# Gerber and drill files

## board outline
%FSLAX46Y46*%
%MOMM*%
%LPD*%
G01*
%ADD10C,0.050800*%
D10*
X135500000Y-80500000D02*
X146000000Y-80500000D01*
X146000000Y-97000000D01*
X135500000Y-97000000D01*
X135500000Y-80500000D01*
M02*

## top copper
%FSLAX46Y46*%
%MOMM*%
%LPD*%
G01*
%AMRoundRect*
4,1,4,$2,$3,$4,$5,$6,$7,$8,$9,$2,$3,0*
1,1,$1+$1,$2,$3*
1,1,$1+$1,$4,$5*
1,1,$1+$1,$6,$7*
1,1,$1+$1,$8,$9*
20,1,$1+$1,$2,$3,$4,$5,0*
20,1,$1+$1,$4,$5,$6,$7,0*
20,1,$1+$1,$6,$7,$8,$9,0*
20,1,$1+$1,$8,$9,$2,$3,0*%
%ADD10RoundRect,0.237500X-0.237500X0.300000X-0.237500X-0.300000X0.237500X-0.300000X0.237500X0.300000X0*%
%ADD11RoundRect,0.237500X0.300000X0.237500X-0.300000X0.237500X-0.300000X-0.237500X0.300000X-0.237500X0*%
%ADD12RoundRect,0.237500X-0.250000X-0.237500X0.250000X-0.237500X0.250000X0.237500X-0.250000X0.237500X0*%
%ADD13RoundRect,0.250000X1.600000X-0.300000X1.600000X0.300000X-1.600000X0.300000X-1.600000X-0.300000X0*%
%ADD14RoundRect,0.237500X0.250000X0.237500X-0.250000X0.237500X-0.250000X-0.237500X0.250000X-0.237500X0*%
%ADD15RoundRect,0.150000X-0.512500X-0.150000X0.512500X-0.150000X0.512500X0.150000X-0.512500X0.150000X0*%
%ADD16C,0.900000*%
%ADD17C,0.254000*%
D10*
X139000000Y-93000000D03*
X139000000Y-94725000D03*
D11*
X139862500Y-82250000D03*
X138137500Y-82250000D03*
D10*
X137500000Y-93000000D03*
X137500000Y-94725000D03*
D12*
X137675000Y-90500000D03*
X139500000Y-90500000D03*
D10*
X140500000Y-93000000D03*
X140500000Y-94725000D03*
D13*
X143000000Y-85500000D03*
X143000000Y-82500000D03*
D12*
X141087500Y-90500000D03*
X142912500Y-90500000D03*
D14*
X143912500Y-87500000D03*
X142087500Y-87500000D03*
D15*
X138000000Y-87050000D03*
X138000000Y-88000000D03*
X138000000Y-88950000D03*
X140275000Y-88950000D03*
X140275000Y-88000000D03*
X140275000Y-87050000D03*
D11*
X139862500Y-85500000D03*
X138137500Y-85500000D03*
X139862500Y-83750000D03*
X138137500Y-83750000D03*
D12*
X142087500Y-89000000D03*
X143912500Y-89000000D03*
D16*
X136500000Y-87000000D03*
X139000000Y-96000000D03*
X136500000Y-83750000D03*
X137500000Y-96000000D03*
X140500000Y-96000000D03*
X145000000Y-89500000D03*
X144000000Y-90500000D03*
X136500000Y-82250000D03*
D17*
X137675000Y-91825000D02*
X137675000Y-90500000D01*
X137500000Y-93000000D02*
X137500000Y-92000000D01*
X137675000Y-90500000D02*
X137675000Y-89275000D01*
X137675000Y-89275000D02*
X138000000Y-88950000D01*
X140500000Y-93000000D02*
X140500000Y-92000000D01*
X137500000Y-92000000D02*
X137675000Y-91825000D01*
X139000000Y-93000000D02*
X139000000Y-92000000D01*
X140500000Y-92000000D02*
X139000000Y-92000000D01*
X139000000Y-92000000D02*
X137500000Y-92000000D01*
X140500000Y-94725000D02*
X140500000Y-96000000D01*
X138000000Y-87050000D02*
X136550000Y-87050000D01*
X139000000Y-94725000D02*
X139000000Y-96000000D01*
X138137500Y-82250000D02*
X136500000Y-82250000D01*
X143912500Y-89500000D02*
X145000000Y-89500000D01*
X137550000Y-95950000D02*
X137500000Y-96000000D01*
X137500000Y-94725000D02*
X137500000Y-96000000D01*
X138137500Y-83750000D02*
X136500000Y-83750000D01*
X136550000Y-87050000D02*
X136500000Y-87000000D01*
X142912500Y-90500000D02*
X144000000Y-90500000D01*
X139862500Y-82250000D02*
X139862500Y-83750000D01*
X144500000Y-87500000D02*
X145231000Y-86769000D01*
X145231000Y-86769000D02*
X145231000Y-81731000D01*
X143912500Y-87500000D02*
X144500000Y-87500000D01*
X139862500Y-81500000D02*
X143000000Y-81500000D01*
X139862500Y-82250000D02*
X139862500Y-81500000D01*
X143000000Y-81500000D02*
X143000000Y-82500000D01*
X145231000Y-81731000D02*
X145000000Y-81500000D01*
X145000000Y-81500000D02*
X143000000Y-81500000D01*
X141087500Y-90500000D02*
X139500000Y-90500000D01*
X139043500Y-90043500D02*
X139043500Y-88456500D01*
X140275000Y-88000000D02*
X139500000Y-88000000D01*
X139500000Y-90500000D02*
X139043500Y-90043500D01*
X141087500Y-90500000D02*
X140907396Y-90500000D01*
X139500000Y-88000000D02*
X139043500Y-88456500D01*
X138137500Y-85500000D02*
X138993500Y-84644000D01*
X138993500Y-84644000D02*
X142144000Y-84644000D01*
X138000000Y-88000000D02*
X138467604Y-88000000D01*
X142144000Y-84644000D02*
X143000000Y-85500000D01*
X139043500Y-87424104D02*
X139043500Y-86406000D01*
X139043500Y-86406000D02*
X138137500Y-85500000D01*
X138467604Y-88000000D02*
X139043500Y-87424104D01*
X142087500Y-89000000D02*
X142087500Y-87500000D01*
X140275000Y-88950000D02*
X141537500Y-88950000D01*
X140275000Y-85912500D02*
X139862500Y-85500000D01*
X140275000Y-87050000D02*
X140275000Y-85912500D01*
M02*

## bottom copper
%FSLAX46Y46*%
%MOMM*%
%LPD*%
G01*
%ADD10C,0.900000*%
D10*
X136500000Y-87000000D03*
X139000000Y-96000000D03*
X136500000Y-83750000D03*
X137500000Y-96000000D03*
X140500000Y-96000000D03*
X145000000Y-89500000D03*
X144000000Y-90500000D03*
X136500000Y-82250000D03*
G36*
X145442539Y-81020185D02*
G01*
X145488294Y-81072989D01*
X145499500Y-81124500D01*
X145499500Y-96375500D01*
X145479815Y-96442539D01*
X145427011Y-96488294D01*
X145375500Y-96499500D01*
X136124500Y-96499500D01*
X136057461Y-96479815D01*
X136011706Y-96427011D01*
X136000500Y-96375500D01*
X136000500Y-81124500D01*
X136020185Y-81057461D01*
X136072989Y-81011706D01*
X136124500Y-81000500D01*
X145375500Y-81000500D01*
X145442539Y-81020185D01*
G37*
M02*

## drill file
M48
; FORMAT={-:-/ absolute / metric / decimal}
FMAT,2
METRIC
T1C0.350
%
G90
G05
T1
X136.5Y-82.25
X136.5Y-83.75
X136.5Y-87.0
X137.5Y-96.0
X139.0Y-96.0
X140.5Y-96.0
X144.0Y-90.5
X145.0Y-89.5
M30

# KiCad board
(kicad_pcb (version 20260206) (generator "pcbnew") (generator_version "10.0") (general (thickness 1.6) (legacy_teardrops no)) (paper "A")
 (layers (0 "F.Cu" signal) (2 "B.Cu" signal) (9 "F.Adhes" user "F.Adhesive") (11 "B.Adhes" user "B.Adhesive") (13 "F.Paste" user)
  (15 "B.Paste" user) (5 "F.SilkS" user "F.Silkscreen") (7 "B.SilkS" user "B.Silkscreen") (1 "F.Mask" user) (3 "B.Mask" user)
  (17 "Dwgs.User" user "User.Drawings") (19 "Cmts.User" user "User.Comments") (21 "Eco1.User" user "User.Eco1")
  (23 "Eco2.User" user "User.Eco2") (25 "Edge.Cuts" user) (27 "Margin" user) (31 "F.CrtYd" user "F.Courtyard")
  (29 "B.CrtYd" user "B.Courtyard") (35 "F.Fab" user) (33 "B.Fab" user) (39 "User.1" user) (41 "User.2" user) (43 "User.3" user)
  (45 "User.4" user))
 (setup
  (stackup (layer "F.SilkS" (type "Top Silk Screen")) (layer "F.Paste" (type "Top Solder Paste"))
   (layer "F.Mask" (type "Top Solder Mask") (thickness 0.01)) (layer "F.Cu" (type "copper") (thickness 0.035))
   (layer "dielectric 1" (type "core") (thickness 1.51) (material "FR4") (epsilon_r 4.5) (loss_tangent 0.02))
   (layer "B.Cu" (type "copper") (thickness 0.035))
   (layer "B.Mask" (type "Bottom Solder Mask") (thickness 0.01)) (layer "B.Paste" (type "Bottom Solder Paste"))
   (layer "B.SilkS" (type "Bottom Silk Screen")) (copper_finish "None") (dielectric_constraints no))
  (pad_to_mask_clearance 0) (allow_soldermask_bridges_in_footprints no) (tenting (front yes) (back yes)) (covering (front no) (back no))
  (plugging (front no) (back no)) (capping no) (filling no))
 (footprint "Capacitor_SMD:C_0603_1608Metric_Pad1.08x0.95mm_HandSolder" (layer "F.Cu") (at 139 93.8625 -90)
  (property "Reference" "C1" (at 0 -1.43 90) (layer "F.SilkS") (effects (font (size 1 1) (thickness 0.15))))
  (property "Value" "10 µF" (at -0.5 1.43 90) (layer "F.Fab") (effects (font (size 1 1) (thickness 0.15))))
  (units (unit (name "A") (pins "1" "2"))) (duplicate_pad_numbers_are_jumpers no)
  (pad "1" smd roundrect (at -0.8625 0 270) (size 1.075 0.95) (layers "F.Cu" "F.Mask" "F.Paste") (roundrect_rratio 0.25) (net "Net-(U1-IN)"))
  (pad "2" smd roundrect (at 0.8625 0 270) (size 1.075 0.95) (layers "F.Cu" "F.Mask" "F.Paste") (roundrect_rratio 0.25) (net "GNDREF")))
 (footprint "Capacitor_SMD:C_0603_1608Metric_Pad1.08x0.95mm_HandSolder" (layer "F.Cu") (at 139 82.25 180)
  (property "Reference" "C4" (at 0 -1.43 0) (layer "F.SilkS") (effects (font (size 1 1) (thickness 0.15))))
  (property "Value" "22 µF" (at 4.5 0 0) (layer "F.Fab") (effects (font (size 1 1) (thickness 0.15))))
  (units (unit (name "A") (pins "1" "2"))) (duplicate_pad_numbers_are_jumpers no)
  (pad "1" smd roundrect (at -0.8625 0 180) (size 1.075 0.95) (layers "F.Cu" "F.Mask" "F.Paste") (roundrect_rratio 0.25)
   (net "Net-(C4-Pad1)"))
  (pad "2" smd roundrect (at 0.8625 0 180) (size 1.075 0.95) (layers "F.Cu" "F.Mask" "F.Paste") (roundrect_rratio 0.25) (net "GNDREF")))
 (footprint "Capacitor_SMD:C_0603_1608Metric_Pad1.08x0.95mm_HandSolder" (layer "F.Cu") (at 137.5 93.8625 -90)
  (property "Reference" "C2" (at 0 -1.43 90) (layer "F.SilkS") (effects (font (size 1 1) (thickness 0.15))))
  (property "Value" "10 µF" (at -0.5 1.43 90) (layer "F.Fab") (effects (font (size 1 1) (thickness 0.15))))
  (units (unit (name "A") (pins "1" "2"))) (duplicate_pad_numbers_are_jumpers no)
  (pad "1" smd roundrect (at -0.8625 0 270) (size 1.075 0.95) (layers "F.Cu" "F.Mask" "F.Paste") (roundrect_rratio 0.25) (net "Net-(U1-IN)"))
  (pad "2" smd roundrect (at 0.8625 0 270) (size 1.075 0.95) (layers "F.Cu" "F.Mask" "F.Paste") (roundrect_rratio 0.25) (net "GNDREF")))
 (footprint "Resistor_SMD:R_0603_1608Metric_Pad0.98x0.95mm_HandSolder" (layer "F.Cu") (at 138.5875 90.5)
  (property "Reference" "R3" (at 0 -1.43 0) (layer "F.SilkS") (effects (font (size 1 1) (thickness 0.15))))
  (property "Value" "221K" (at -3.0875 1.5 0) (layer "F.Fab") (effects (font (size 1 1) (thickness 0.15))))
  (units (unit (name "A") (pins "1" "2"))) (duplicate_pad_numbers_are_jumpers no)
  (pad "1" smd roundrect (at -0.9125 0) (size 0.975 0.95) (layers "F.Cu" "F.Mask" "F.Paste") (roundrect_rratio 0.25) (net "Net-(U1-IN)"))
  (pad "2" smd roundrect (at 0.9125 0) (size 0.975 0.95) (layers "F.Cu" "F.Mask" "F.Paste") (roundrect_rratio 0.25) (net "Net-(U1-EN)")))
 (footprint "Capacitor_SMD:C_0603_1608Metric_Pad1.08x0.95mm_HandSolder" (layer "F.Cu") (at 140.5 93.8625 -90)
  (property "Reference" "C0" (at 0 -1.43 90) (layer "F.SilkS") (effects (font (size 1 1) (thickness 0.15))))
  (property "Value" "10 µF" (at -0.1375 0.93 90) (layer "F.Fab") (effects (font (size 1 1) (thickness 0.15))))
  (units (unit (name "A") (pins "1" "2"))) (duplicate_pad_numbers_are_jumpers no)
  (pad "1" smd roundrect (at -0.8625 0 270) (size 1.075 0.95) (layers "F.Cu" "F.Mask" "F.Paste") (roundrect_rratio 0.25) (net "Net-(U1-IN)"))
  (pad "2" smd roundrect (at 0.8625 0 270) (size 1.075 0.95) (layers "F.Cu" "F.Mask" "F.Paste") (roundrect_rratio 0.25) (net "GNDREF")))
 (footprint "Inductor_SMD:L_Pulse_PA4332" (layer "F.Cu") (at 143 84 90)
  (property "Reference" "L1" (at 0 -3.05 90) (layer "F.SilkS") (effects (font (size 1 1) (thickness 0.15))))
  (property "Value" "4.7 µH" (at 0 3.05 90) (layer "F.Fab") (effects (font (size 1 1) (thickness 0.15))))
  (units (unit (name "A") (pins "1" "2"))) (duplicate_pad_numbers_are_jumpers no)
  (pad "1" smd roundrect (at -1.5 0 90) (size 1.1 3.7) (layers "F.Cu" "F.Mask" "F.Paste") (roundrect_rratio 0.227273) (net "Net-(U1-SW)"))
  (pad "2" smd roundrect (at 1.5 0 90) (size 1.1 3.7) (layers "F.Cu" "F.Mask" "F.Paste") (roundrect_rratio 0.227273) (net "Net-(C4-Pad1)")))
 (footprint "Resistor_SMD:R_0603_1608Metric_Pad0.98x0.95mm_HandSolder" (layer "F.Cu") (at 142 90.5)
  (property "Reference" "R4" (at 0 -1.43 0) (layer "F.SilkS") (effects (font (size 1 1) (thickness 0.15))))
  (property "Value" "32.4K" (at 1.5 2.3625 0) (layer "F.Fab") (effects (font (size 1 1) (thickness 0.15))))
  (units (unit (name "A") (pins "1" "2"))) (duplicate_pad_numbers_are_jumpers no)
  (pad "1" smd roundrect (at -0.9125 0) (size 0.975 0.95) (layers "F.Cu" "F.Mask" "F.Paste") (roundrect_rratio 0.25) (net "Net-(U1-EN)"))
  (pad "2" smd roundrect (at 0.9125 0) (size 0.975 0.95) (layers "F.Cu" "F.Mask" "F.Paste") (roundrect_rratio 0.25) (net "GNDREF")))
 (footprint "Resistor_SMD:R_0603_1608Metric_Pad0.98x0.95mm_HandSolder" (layer "F.Cu") (at 143 87.5 180)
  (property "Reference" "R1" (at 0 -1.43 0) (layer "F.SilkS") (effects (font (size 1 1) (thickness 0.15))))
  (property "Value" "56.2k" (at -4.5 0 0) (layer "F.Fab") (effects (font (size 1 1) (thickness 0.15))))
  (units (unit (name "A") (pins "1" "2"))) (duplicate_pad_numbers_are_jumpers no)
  (pad "1" smd roundrect (at -0.9125 0 180) (size 0.975 0.95) (layers "F.Cu" "F.Mask" "F.Paste") (roundrect_rratio 0.25)
   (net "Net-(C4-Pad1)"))
  (pad "2" smd roundrect (at 0.9125 0 180) (size 0.975 0.95) (layers "F.Cu" "F.Mask" "F.Paste") (roundrect_rratio 0.25) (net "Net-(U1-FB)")))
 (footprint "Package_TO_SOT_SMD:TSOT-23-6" (layer "F.Cu") (at 139.1375 88)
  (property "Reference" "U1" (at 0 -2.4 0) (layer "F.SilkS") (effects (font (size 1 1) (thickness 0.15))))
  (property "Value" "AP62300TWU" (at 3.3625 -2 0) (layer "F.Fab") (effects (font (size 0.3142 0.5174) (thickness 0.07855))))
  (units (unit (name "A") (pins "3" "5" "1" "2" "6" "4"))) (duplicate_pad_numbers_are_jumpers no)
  (pad "1" smd roundrect (at -1.1375 -0.95) (size 1.325 0.6) (layers "F.Cu" "F.Mask" "F.Paste") (roundrect_rratio 0.25) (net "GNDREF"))
  (pad "2" smd roundrect (at -1.1375 0) (size 1.325 0.6) (layers "F.Cu" "F.Mask" "F.Paste") (roundrect_rratio 0.25) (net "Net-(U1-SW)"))
  (pad "3" smd roundrect (at -1.1375 0.95) (size 1.325 0.6) (layers "F.Cu" "F.Mask" "F.Paste") (roundrect_rratio 0.25) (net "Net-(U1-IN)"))
  (pad "4" smd roundrect (at 1.1375 0.95) (size 1.325 0.6) (layers "F.Cu" "F.Mask" "F.Paste") (roundrect_rratio 0.25) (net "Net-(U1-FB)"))
  (pad "5" smd roundrect (at 1.1375 0) (size 1.325 0.6) (layers "F.Cu" "F.Mask" "F.Paste") (roundrect_rratio 0.25) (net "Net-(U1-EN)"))
  (pad "6" smd roundrect (at 1.1375 -0.95) (size 1.325 0.6) (layers "F.Cu" "F.Mask" "F.Paste") (roundrect_rratio 0.25) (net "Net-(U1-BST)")))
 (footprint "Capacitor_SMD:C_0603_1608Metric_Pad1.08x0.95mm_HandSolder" (layer "F.Cu") (at 139 85.5 180)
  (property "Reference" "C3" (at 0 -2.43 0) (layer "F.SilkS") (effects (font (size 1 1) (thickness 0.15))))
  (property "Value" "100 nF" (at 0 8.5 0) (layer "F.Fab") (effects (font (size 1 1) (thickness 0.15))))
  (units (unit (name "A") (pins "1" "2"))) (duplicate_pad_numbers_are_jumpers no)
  (pad "1" smd roundrect (at -0.8625 0 180) (size 1.075 0.95) (layers "F.Cu" "F.Mask" "F.Paste") (roundrect_rratio 0.25)
   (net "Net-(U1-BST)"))
  (pad "2" smd roundrect (at 0.8625 0 180) (size 1.075 0.95) (layers "F.Cu" "F.Mask" "F.Paste") (roundrect_rratio 0.25) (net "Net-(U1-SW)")))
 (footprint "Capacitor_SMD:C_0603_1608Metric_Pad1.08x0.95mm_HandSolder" (layer "F.Cu") (at 139 83.75 180)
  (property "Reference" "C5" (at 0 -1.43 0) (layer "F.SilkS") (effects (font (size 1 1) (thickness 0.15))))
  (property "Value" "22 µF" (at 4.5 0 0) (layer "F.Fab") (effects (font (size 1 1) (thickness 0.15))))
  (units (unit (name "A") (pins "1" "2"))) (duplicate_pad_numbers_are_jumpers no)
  (pad "1" smd roundrect (at -0.8625 0 180) (size 1.075 0.95) (layers "F.Cu" "F.Mask" "F.Paste") (roundrect_rratio 0.25)
   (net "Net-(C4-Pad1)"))
  (pad "2" smd roundrect (at 0.8625 0 180) (size 1.075 0.95) (layers "F.Cu" "F.Mask" "F.Paste") (roundrect_rratio 0.25) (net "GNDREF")))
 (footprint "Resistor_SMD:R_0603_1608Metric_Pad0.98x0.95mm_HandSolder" (layer "F.Cu") (at 143 89)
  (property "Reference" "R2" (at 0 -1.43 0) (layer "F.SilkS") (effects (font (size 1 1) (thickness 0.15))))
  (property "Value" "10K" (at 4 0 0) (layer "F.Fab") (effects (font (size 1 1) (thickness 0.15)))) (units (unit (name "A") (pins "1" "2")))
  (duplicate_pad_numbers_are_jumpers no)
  (pad "1" smd roundrect (at -0.9125 0) (size 0.975 0.95) (layers "F.Cu" "F.Mask" "F.Paste") (roundrect_rratio 0.25) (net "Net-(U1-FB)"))
  (pad "2" smd roundrect (at 0.9125 0) (size 0.975 0.95) (layers "F.Cu" "F.Mask" "F.Paste") (roundrect_rratio 0.25) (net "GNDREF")))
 (gr_rect (start 135.5 80.5) (end 146 97) (stroke (width 0.0508) (type solid)) (fill no) (layer "Edge.Cuts"))
 (segment (start 137.675 91.825) (end 137.675 90.5) (width 0.254) (layer "F.Cu") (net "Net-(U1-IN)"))
 (segment (start 137.5 93) (end 137.5 92) (width 0.254) (layer "F.Cu") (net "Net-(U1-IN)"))
 (segment (start 137.675 90.5) (end 137.675 89.275) (width 0.254) (layer "F.Cu") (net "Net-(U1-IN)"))
 (segment (start 137.675 89.275) (end 138 88.95) (width 0.254) (layer "F.Cu") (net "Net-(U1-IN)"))
 (segment (start 140.5 93) (end 140.5 92) (width 0.254) (layer "F.Cu") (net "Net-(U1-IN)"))
 (segment (start 137.5 92) (end 137.675 91.825) (width 0.254) (layer "F.Cu") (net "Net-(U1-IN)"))
 (segment (start 139 93) (end 139 92) (width 0.254) (layer "F.Cu") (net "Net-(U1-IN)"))
 (segment (start 140.5 92) (end 139 92) (width 0.254) (layer "F.Cu") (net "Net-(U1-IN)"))
 (segment (start 139 92) (end 137.5 92) (width 0.254) (layer "F.Cu") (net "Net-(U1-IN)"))
 (segment (start 140.5 94.725) (end 140.5 96) (width 0.254) (layer "F.Cu") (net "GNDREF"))
 (segment (start 138 87.05) (end 136.55 87.05) (width 0.254) (layer "F.Cu") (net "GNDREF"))
 (segment (start 139 94.725) (end 139 96) (width 0.254) (layer "F.Cu") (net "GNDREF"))
 (segment (start 138.1375 82.25) (end 136.5 82.25) (width 0.254) (layer "F.Cu") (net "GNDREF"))
 (segment (start 143.9125 89.5) (end 145 89.5) (width 0.254) (layer "F.Cu") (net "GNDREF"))
 (segment (start 137.55 95.95) (end 137.5 96) (width 0.254) (layer "F.Cu") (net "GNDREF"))
 (segment (start 137.5 94.725) (end 137.5 96) (width 0.254) (layer "F.Cu") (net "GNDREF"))
 (segment (start 138.1375 83.75) (end 136.5 83.75) (width 0.254) (layer "F.Cu") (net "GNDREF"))
 (segment (start 136.55 87.05) (end 136.5 87) (width 0.254) (layer "F.Cu") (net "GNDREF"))
 (segment (start 142.9125 90.5) (end 144 90.5) (width 0.254) (layer "F.Cu") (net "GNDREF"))
 (via (at 136.5 87) (size 0.9) (drill 0.35) (layers "F.Cu" "B.Cu") (free yes) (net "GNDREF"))
 (via (at 139 96) (size 0.9) (drill 0.35) (layers "F.Cu" "B.Cu") (free yes) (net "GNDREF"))
 (via (at 136.5 83.75) (size 0.9) (drill 0.35) (layers "F.Cu" "B.Cu") (free yes) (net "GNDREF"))
 (via (at 137.5 96) (size 0.9) (drill 0.35) (layers "F.Cu" "B.Cu") (free yes) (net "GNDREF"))
 (via (at 140.5 96) (size 0.9) (drill 0.35) (layers "F.Cu" "B.Cu") (free yes) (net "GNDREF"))
 (via (at 145 89.5) (size 0.9) (drill 0.35) (layers "F.Cu" "B.Cu") (free yes) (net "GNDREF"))
 (via (at 144 90.5) (size 0.9) (drill 0.35) (layers "F.Cu" "B.Cu") (free yes) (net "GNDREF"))
 (via (at 136.5 82.25) (size 0.9) (drill 0.35) (layers "F.Cu" "B.Cu") (free yes) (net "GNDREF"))
 (segment (start 139.8625 82.25) (end 139.8625 83.75) (width 0.254) (layer "F.Cu") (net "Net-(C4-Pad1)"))
 (segment (start 144.5 87.5) (end 145.231 86.769) (width 0.254) (layer "F.Cu") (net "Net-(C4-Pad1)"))
 (segment (start 145.231 86.769) (end 145.231 81.731) (width 0.254) (layer "F.Cu") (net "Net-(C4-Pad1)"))
 (segment (start 143.9125 87.5) (end 144.5 87.5) (width 0.254) (layer "F.Cu") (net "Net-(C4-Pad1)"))
 (segment (start 139.8625 81.5) (end 143 81.5) (width 0.254) (layer "F.Cu") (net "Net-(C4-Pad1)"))
 (segment (start 139.8625 82.25) (end 139.8625 81.5) (width 0.254) (layer "F.Cu") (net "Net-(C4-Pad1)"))
 (segment (start 143 81.5) (end 143 82.5) (width 0.254) (layer "F.Cu") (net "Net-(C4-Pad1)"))
 (segment (start 145.231 81.731) (end 145 81.5) (width 0.254) (layer "F.Cu") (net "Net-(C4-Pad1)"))
 (segment (start 145 81.5) (end 143 81.5) (width 0.254) (layer "F.Cu") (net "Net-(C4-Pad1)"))
 (segment (start 141.0875 90.5) (end 139.5 90.5) (width 0.254) (layer "F.Cu") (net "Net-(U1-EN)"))
 (segment (start 139.0435 90.0435) (end 139.0435 88.4565) (width 0.254) (layer "F.Cu") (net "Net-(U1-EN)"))
 (segment (start 140.275 88) (end 139.5 88) (width 0.254) (layer "F.Cu") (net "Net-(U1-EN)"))
 (segment (start 139.5 90.5) (end 139.0435 90.0435) (width 0.254) (layer "F.Cu") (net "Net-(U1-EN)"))
 (segment (start 141.0875 90.5) (end 140.907396 90.5) (width 0.254) (layer "F.Cu") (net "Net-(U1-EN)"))
 (segment (start 139.5 88) (end 139.0435 88.4565) (width 0.254) (layer "F.Cu") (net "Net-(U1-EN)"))
 (segment (start 138.1375 85.5) (end 138.9935 84.644) (width 0.254) (layer "F.Cu") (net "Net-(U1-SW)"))
 (segment (start 138.9935 84.644) (end 142.144 84.644) (width 0.254) (layer "F.Cu") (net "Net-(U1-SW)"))
 (segment (start 138 88) (end 138.467604 88) (width 0.254) (layer "F.Cu") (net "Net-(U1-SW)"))
 (segment (start 142.144 84.644) (end 143 85.5) (width 0.254) (layer "F.Cu") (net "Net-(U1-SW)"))
 (segment (start 139.0435 87.424104) (end 139.0435 86.406) (width 0.254) (layer "F.Cu") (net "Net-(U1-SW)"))
 (segment (start 139.0435 86.406) (end 138.1375 85.5) (width 0.254) (layer "F.Cu") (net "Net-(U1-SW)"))
 (segment (start 138.467604 88) (end 139.0435 87.424104) (width 0.254) (layer "F.Cu") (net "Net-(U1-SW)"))
 (segment (start 142.0875 89) (end 142.0875 87.5) (width 0.254) (layer "F.Cu") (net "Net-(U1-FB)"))
 (segment (start 140.275 88.95) (end 141.5375 88.95) (width 0.254) (layer "F.Cu") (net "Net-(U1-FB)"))
 (segment (start 140.275 85.9125) (end 139.8625 85.5) (width 0.254) (layer "F.Cu") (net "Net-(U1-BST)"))
 (segment (start 140.275 87.05) (end 140.275 85.9125) (width 0.254) (layer "F.Cu") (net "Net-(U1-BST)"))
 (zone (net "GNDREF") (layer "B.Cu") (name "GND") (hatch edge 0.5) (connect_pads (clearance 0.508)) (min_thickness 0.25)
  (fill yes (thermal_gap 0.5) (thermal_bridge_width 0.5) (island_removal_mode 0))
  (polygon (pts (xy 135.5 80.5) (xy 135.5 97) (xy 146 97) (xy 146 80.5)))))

